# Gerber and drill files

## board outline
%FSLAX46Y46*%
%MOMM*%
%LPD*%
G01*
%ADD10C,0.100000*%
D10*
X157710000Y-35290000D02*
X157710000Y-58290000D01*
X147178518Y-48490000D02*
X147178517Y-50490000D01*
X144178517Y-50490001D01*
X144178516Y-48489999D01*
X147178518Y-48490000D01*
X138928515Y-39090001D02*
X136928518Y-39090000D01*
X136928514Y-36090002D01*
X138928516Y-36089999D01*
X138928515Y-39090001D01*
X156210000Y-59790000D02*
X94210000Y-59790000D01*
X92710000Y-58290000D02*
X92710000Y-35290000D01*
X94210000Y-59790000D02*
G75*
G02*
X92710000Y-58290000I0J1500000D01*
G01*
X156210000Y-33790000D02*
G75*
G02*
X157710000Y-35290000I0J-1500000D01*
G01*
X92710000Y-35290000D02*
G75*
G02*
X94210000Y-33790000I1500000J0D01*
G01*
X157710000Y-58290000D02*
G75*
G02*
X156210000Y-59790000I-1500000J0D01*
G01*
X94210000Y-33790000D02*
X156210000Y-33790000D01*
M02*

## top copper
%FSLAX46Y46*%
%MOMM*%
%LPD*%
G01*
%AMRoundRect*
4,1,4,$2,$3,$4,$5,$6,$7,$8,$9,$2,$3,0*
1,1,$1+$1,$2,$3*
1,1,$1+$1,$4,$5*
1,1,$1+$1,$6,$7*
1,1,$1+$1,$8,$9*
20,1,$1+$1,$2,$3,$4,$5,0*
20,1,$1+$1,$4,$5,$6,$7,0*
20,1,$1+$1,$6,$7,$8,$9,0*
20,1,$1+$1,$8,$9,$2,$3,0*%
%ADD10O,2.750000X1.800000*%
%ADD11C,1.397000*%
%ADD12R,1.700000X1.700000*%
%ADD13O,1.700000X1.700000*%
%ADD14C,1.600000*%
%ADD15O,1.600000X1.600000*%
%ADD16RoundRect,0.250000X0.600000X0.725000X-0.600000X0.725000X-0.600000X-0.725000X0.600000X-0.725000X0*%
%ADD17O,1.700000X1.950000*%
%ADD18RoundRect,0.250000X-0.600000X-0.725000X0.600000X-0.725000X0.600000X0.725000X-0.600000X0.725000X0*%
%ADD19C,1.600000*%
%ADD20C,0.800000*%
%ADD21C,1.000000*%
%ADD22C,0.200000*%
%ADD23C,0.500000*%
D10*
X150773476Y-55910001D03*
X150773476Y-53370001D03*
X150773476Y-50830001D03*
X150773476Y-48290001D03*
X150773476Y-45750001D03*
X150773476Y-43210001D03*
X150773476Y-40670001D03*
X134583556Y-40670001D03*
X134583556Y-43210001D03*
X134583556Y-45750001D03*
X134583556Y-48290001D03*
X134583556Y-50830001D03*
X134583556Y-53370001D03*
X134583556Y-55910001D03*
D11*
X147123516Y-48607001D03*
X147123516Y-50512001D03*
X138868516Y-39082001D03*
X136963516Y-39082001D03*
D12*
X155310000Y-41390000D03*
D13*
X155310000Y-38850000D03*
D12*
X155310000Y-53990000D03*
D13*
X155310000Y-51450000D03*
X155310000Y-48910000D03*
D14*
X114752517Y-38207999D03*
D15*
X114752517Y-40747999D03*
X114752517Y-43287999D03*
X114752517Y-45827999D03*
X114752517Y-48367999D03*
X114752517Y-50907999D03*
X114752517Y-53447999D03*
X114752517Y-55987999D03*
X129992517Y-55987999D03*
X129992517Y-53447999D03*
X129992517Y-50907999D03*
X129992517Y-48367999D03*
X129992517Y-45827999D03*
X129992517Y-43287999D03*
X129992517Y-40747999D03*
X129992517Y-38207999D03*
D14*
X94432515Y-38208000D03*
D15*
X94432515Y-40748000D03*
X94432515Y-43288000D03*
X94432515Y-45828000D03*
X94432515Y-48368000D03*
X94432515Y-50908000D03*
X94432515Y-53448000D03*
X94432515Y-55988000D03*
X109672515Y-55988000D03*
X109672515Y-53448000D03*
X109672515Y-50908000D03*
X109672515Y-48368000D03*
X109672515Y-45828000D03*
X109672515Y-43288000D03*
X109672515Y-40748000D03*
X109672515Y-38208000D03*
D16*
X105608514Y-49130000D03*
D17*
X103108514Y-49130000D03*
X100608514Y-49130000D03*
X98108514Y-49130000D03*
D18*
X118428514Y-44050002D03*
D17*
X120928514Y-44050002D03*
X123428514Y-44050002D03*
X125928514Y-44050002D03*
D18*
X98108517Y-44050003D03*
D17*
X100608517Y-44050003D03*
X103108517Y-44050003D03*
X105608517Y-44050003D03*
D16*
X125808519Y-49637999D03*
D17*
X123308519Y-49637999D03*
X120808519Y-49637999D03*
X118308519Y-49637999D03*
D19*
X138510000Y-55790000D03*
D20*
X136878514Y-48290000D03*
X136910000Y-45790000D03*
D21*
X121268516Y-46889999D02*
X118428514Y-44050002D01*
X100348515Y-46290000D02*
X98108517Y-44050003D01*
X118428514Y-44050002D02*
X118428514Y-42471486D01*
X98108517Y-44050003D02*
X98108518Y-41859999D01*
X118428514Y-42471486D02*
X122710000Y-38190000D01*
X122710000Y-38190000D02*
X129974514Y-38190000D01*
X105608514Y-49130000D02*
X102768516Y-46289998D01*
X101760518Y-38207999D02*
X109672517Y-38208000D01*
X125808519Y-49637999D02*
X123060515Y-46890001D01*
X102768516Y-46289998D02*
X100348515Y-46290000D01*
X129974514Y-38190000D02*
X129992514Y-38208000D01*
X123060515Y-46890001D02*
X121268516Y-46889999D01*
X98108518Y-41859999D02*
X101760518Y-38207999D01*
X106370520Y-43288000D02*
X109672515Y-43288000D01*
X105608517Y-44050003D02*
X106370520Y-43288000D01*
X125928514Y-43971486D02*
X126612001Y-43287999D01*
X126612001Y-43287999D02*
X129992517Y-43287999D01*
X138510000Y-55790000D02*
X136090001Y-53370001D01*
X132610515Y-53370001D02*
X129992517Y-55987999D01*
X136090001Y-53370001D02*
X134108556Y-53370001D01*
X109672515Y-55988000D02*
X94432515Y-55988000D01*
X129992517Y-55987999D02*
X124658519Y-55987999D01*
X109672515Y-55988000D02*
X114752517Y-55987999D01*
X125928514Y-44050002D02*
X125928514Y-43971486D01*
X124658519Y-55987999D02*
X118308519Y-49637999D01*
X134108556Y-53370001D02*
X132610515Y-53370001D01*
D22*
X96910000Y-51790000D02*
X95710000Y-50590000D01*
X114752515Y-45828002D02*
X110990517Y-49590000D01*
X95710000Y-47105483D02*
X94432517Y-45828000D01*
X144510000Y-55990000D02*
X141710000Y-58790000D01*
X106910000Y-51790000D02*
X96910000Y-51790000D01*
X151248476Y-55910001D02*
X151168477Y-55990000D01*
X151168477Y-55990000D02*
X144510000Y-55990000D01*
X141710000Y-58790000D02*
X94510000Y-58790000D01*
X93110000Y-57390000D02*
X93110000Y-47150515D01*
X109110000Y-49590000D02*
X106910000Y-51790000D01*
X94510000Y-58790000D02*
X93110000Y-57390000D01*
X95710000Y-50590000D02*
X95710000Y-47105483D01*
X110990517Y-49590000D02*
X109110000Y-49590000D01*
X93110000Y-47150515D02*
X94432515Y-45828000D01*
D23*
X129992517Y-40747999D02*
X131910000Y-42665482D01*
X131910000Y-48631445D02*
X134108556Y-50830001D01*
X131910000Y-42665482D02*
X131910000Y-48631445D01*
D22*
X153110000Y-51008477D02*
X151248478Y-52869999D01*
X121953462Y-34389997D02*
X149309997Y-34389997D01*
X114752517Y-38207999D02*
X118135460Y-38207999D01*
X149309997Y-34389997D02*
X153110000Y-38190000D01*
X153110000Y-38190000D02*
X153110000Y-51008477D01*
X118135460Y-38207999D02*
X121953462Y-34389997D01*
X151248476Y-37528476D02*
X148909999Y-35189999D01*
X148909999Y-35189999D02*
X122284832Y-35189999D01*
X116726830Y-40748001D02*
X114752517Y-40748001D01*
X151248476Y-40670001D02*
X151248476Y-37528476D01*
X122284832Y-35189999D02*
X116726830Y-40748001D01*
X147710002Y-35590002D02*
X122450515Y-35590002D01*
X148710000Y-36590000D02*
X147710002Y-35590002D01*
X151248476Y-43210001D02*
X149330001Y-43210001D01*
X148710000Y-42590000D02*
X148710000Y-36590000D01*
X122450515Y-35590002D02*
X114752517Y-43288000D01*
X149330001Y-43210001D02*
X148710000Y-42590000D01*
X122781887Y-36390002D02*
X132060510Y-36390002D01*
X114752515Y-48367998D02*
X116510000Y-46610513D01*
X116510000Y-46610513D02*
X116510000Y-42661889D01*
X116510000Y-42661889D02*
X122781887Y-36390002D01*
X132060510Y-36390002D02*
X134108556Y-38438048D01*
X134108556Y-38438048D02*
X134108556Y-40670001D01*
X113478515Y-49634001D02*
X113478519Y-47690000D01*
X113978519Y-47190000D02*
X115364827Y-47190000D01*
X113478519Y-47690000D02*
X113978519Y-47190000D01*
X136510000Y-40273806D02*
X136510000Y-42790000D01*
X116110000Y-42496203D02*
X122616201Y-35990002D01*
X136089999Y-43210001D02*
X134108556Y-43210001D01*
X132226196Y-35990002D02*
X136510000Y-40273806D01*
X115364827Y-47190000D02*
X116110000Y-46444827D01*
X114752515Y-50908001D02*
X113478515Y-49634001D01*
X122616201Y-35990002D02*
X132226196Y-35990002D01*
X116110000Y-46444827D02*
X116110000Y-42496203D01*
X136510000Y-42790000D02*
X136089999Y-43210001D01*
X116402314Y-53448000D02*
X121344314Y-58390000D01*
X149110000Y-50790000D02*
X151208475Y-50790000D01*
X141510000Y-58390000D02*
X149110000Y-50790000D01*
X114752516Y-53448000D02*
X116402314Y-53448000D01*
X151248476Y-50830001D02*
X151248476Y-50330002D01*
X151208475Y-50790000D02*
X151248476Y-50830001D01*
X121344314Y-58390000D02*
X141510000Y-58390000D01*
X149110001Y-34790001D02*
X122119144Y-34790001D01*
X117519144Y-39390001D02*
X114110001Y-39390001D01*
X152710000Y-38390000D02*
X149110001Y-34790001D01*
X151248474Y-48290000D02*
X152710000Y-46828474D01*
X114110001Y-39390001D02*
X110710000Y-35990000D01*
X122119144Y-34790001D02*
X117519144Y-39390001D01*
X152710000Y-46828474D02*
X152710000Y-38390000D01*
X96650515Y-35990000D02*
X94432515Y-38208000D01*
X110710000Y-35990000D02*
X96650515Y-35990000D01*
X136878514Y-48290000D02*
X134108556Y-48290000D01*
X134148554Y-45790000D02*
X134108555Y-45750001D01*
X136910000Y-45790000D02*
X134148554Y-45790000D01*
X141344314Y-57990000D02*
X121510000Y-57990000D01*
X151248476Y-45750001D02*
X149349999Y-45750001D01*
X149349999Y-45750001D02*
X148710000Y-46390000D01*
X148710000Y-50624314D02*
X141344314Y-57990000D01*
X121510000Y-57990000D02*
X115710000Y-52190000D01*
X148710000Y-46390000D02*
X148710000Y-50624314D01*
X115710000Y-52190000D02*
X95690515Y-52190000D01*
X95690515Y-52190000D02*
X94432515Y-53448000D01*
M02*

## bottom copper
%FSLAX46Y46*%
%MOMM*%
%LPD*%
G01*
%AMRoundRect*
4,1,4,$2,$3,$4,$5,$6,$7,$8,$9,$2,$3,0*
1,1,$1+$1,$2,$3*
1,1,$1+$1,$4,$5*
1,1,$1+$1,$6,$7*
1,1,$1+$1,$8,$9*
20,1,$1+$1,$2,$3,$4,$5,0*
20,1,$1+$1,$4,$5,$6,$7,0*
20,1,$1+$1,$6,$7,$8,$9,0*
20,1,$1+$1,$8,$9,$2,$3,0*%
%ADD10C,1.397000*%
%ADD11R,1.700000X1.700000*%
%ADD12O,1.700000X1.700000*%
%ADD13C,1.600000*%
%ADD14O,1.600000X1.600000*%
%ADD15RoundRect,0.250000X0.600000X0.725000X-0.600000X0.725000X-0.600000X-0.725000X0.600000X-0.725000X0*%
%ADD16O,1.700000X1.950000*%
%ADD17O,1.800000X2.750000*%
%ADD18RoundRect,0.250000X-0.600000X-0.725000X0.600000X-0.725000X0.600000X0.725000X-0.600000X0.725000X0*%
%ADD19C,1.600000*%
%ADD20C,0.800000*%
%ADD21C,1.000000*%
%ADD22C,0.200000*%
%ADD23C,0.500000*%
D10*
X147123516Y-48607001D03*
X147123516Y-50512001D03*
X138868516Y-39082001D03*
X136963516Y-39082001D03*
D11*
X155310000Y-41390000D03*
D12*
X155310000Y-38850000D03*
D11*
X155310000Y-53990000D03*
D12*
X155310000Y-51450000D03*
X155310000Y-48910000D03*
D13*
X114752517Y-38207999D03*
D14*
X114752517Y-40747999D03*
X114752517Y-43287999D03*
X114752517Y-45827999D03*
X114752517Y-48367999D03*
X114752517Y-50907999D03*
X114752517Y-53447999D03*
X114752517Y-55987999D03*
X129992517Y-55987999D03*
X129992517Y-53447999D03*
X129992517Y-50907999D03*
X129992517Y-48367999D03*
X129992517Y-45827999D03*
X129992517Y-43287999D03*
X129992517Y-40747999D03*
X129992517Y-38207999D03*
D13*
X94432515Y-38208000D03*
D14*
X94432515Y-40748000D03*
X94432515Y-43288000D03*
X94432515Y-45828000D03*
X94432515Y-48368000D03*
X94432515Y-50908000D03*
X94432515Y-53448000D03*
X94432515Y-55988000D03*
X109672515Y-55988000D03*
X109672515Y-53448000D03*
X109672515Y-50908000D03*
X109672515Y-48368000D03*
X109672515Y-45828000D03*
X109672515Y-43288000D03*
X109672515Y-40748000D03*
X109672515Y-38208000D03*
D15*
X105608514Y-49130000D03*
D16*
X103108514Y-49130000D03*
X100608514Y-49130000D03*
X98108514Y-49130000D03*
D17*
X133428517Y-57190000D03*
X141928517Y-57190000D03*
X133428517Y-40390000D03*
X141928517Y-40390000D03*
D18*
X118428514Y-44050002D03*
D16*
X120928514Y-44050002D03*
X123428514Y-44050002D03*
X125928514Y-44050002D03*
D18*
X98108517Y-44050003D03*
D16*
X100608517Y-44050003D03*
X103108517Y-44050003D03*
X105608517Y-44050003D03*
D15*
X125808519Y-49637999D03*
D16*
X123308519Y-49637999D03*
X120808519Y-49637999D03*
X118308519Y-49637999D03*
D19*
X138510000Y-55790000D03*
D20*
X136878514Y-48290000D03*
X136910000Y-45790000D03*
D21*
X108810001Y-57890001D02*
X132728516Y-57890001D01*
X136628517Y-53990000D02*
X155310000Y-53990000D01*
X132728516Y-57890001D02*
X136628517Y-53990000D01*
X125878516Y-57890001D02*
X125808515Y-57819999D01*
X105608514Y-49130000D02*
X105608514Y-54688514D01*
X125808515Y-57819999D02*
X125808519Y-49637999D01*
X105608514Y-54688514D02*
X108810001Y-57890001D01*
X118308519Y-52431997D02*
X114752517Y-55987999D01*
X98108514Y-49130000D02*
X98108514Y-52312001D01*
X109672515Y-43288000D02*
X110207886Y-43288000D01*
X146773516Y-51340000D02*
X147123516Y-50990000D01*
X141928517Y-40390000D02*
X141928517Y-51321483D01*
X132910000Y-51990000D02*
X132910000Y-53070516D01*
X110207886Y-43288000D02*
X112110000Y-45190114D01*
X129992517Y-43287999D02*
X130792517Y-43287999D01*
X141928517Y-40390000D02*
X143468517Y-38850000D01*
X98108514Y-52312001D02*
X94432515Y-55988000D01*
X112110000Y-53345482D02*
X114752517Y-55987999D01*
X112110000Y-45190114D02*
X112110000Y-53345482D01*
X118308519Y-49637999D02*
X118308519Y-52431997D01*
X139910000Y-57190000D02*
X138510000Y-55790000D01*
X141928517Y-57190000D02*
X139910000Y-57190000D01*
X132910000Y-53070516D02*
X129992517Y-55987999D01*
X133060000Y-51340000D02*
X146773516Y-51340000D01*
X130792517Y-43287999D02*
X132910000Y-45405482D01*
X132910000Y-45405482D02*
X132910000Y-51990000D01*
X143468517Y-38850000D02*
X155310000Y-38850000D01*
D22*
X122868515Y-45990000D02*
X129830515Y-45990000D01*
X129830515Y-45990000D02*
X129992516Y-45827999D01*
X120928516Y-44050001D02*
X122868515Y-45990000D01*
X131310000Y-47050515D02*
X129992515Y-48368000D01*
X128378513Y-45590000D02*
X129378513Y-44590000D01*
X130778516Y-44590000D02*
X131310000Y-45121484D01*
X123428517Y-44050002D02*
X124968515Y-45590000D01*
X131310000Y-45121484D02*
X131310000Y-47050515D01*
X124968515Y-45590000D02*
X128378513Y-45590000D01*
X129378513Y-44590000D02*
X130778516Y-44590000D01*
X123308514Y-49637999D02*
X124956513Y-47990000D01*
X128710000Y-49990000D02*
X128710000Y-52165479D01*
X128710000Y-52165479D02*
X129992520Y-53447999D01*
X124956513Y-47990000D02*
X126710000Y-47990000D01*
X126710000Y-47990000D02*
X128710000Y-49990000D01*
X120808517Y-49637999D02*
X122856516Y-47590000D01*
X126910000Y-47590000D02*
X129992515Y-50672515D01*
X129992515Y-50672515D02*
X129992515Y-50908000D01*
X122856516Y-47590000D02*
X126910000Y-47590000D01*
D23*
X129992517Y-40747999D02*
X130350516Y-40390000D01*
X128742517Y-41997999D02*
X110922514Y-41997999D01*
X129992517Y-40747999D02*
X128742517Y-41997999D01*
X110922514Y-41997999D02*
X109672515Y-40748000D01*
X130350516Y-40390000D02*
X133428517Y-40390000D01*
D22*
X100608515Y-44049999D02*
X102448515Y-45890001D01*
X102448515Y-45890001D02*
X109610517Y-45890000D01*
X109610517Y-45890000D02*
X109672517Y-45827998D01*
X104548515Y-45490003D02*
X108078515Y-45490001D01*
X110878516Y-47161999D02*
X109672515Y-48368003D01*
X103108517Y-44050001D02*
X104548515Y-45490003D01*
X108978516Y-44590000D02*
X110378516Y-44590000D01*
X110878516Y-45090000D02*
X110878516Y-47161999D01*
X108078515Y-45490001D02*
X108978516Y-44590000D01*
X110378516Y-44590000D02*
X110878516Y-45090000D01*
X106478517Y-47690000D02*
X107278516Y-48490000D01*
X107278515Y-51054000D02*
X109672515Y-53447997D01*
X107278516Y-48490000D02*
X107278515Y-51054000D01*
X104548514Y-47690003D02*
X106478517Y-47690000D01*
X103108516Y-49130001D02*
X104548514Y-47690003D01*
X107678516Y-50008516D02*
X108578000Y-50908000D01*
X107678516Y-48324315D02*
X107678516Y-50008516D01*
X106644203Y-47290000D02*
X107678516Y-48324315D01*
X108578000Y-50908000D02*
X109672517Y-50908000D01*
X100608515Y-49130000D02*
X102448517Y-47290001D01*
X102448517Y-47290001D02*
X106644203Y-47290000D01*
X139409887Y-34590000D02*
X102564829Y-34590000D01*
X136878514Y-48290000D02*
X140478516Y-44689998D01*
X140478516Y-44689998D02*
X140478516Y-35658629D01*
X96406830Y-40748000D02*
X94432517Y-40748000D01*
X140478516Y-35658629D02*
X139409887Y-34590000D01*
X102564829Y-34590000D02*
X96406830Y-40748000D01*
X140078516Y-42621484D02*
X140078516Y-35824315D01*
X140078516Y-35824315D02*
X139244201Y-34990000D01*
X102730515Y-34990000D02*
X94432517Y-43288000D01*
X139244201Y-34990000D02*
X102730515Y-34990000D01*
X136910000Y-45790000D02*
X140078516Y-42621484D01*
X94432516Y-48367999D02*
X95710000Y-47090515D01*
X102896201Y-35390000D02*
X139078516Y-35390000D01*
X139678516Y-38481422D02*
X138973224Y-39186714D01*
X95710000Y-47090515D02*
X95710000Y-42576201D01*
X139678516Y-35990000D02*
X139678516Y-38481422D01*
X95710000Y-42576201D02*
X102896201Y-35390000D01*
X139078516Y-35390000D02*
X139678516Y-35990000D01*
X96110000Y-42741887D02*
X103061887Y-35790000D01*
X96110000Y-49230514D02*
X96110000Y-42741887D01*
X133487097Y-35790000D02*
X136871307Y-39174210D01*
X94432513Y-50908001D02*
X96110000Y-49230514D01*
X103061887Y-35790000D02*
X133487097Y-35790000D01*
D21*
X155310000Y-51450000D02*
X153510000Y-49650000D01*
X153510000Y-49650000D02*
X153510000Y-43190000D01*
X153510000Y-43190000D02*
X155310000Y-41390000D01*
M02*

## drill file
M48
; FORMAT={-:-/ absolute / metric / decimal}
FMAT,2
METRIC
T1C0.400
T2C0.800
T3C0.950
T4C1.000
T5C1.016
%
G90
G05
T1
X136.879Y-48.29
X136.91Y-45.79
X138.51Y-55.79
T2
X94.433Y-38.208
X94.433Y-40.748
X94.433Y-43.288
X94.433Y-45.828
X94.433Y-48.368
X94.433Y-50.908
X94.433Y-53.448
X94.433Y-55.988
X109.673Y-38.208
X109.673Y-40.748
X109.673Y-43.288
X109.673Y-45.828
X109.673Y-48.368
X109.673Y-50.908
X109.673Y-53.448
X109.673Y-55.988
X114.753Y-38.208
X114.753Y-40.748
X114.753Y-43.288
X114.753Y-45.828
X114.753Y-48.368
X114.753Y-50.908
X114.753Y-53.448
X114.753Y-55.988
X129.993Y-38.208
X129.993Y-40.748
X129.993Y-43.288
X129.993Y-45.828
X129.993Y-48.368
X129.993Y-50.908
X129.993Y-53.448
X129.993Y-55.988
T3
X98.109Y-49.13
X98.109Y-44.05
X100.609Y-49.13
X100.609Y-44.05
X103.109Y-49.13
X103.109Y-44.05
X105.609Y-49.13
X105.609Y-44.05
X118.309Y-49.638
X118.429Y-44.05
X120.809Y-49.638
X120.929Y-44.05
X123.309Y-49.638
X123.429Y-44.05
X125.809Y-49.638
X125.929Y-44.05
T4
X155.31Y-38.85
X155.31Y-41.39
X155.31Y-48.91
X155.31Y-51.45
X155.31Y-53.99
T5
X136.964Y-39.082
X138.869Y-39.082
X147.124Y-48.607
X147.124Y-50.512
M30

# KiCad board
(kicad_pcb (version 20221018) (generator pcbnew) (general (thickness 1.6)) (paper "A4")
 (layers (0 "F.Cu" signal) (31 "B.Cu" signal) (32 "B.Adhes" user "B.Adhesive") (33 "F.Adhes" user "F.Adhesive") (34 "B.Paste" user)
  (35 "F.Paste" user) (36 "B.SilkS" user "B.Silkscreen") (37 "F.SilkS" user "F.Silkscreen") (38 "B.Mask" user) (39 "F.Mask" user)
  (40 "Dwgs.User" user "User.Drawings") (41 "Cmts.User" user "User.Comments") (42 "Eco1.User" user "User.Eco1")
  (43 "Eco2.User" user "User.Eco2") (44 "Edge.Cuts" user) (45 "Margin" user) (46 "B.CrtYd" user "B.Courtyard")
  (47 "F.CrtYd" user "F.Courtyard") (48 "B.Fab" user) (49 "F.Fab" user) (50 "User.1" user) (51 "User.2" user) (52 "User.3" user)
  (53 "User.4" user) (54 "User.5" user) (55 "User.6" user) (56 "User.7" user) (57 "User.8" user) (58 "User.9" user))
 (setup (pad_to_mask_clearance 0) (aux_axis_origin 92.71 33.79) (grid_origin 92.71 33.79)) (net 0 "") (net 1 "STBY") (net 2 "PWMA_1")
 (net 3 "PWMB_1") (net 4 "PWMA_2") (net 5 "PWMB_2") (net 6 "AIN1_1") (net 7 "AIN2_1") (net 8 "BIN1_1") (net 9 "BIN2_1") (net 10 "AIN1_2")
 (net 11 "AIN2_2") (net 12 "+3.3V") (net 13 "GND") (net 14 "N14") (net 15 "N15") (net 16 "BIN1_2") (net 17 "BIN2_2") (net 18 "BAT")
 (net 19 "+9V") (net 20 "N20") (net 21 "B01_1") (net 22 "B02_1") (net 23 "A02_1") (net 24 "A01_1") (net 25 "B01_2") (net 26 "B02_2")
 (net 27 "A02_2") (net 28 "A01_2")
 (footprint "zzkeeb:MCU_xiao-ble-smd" (layer "F.Cu") (at 142.678516 48.290001 180)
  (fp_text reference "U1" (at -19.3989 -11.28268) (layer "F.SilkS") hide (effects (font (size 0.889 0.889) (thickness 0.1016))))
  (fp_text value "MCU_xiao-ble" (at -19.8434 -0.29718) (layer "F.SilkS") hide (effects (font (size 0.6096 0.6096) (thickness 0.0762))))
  (pad "1" smd oval (at -8.56996 -7.62) (size 2.75 1.8) (drill (offset -0.475 0)) (layers "F.Cu" "F.Paste" "F.Mask") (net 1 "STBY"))
  (pad "2" smd oval (at -8.56996 -5.08) (size 2.75 1.8) (drill (offset -0.475 0)) (layers "F.Cu" "F.Paste" "F.Mask") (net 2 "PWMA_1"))
  (pad "3" smd oval (at -8.56996 -2.54) (size 2.75 1.8) (drill (offset -0.475 0)) (layers "F.Cu" "F.Paste" "F.Mask") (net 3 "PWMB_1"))
  (pad "4" smd oval (at -8.56996 0) (size 2.75 1.8) (drill (offset -0.475 0)) (layers "F.Cu" "F.Paste" "F.Mask") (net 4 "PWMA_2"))
  (pad "5" smd oval (at -8.56996 2.54) (size 2.75 1.8) (drill (offset -0.475 0)) (layers "F.Cu" "F.Paste" "F.Mask") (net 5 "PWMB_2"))
  (pad "6" smd oval (at -8.56996 5.08) (size 2.75 1.8) (drill (offset -0.475 0)) (layers "F.Cu" "F.Paste" "F.Mask") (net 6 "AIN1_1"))
  (pad "7" smd oval (at -8.56996 7.62) (size 2.75 1.8) (drill (offset -0.475 0)) (layers "F.Cu" "F.Paste" "F.Mask") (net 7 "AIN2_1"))
  (pad "8" smd oval (at 8.56996 7.62 180) (size 2.75 1.8) (drill (offset -0.475 0)) (layers "F.Cu" "F.Paste" "F.Mask") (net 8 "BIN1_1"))
  (pad "9" smd oval (at 8.56996 5.08 180) (size 2.75 1.8) (drill (offset -0.475 0)) (layers "F.Cu" "F.Paste" "F.Mask") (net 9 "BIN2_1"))
  (pad "10" smd oval (at 8.56996 2.54 180) (size 2.75 1.8) (drill (offset -0.475 0)) (layers "F.Cu" "F.Paste" "F.Mask") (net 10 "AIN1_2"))
  (pad "11" smd oval (at 8.56996 0 180) (size 2.75 1.8) (drill (offset -0.475 0)) (layers "F.Cu" "F.Paste" "F.Mask") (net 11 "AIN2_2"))
  (pad "12" smd oval (at 8.56996 -2.54 180) (size 2.75 1.8) (drill (offset -0.475 0)) (layers "F.Cu" "F.Paste" "F.Mask") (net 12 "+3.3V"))
  (pad "13" smd oval (at 8.56996 -5.08 180) (size 2.75 1.8) (drill (offset -0.475 0)) (layers "F.Cu" "F.Paste" "F.Mask") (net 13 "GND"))
  (pad "14" smd oval (at 8.56996 -7.62 180) (size 2.75 1.8) (drill (offset -0.475 0)) (layers "F.Cu" "F.Paste" "F.Mask") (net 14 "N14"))
  (pad "19" thru_hole circle (at -4.445 -0.317) (size 1.397 1.397) (drill 1.016) (layers "*.Cu" "*.Mask") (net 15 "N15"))
  (pad "20" thru_hole circle (at -4.445 -2.222) (size 1.397 1.397) (drill 1.016) (layers "*.Cu" "*.Mask") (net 13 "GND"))
  (pad "21" thru_hole circle (at 3.81 9.208) (size 1.397 1.397) (drill 1.016) (layers "*.Cu" "*.Mask") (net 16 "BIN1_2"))
  (pad "22" thru_hole circle (at 5.715 9.208) (size 1.397 1.397) (drill 1.016) (layers "*.Cu" "*.Mask") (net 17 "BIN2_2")))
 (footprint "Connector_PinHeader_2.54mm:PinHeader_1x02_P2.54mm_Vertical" (layer "F.Cu") (at 155.31 41.39 180)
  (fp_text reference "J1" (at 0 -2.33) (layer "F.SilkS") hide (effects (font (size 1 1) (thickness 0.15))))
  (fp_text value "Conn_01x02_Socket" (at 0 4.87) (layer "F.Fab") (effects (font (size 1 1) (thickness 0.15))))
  (pad "1" thru_hole rect (at 0 0 180) (size 1.7 1.7) (drill 1) (layers "*.Cu" "*.Mask") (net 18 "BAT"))
  (pad "2" thru_hole oval (at 0 2.54 180) (size 1.7 1.7) (drill 1) (layers "*.Cu" "*.Mask") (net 13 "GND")))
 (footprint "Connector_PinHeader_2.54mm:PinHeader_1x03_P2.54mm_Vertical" (layer "F.Cu") (at 155.31 53.99 180)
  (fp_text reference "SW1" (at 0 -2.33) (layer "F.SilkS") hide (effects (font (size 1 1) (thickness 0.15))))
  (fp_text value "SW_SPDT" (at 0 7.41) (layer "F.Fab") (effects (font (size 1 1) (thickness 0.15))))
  (pad "1" thru_hole rect (at 0 0 180) (size 1.7 1.7) (drill 1) (layers "*.Cu" "*.Mask") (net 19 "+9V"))
  (pad "2" thru_hole oval (at 0 2.54 180) (size 1.7 1.7) (drill 1) (layers "*.Cu" "*.Mask") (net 18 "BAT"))
  (pad "3" thru_hole oval (at 0 5.08 180) (size 1.7 1.7) (drill 1) (layers "*.Cu" "*.Mask") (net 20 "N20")))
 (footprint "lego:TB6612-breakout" (layer "F.Cu") (at 114.752517 38.207999)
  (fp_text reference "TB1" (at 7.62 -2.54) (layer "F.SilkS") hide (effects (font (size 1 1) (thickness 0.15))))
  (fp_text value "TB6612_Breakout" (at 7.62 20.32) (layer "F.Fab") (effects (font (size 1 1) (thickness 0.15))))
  (pad "1" thru_hole circle (at 0 0) (size 1.6 1.6) (drill 0.8) (layers "*.Cu" "*.Mask") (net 2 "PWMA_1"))
  (pad "2" thru_hole oval (at 0 2.54) (size 1.6 1.6) (drill 0.8) (layers "*.Cu" "*.Mask") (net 7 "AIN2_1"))
  (pad "3" thru_hole oval (at 0 5.08) (size 1.6 1.6) (drill 0.8) (layers "*.Cu" "*.Mask") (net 6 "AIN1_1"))
  (pad "4" thru_hole oval (at 0 7.62) (size 1.6 1.6) (drill 0.8) (layers "*.Cu" "*.Mask") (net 1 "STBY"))
  (pad "5" thru_hole oval (at 0 10.16) (size 1.6 1.6) (drill 0.8) (layers "*.Cu" "*.Mask") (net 8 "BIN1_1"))
  (pad "6" thru_hole oval (at 0 12.7) (size 1.6 1.6) (drill 0.8) (layers "*.Cu" "*.Mask") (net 9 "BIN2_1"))
  (pad "7" thru_hole oval (at 0 15.24) (size 1.6 1.6) (drill 0.8) (layers "*.Cu" "*.Mask") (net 3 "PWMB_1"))
  (pad "8" thru_hole oval (at 0 17.78) (size 1.6 1.6) (drill 0.8) (layers "*.Cu" "*.Mask") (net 13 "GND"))
  (pad "9" thru_hole oval (at 15.24 17.78) (size 1.6 1.6) (drill 0.8) (layers "*.Cu" "*.Mask") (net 13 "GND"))
  (pad "10" thru_hole oval (at 15.24 15.24) (size 1.6 1.6) (drill 0.8) (layers "*.Cu" "*.Mask") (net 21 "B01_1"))
  (pad "11" thru_hole oval (at 15.24 12.7) (size 1.6 1.6) (drill 0.8) (layers "*.Cu" "*.Mask") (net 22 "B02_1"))
  (pad "12" thru_hole oval (at 15.24 10.16) (size 1.6 1.6) (drill 0.8) (layers "*.Cu" "*.Mask") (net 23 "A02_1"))
  (pad "13" thru_hole oval (at 15.24 7.62) (size 1.6 1.6) (drill 0.8) (layers "*.Cu" "*.Mask") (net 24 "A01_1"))
  (pad "14" thru_hole oval (at 15.24 5.08) (size 1.6 1.6) (drill 0.8) (layers "*.Cu" "*.Mask") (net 13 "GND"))
  (pad "15" thru_hole oval (at 15.24 2.54) (size 1.6 1.6) (drill 0.8) (layers "*.Cu" "*.Mask") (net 12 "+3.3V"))
  (pad "16" thru_hole oval (at 15.24 0) (size 1.6 1.6) (drill 0.8) (layers "*.Cu" "*.Mask") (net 19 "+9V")))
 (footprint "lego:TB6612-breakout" (layer "F.Cu") (at 94.432515 38.208)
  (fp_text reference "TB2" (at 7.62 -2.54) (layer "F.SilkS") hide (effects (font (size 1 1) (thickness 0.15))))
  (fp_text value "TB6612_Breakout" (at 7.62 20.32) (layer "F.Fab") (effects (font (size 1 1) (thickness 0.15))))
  (pad "1" thru_hole circle (at 0 0) (size 1.6 1.6) (drill 0.8) (layers "*.Cu" "*.Mask") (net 4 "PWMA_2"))
  (pad "2" thru_hole oval (at 0 2.54) (size 1.6 1.6) (drill 0.8) (layers "*.Cu" "*.Mask") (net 11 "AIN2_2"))
  (pad "3" thru_hole oval (at 0 5.08) (size 1.6 1.6) (drill 0.8) (layers "*.Cu" "*.Mask") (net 10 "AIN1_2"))
  (pad "4" thru_hole oval (at 0 7.62) (size 1.6 1.6) (drill 0.8) (layers "*.Cu" "*.Mask") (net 1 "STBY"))
  (pad "5" thru_hole oval (at 0 10.16) (size 1.6 1.6) (drill 0.8) (layers "*.Cu" "*.Mask") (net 16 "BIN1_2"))
  (pad "6" thru_hole oval (at 0 12.7) (size 1.6 1.6) (drill 0.8) (layers "*.Cu" "*.Mask") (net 17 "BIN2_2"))
  (pad "7" thru_hole oval (at 0 15.24) (size 1.6 1.6) (drill 0.8) (layers "*.Cu" "*.Mask") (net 5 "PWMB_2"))
  (pad "8" thru_hole oval (at 0 17.78) (size 1.6 1.6) (drill 0.8) (layers "*.Cu" "*.Mask") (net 13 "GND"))
  (pad "9" thru_hole oval (at 15.24 17.78) (size 1.6 1.6) (drill 0.8) (layers "*.Cu" "*.Mask") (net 13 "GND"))
  (pad "10" thru_hole oval (at 15.24 15.24) (size 1.6 1.6) (drill 0.8) (layers "*.Cu" "*.Mask") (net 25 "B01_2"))
  (pad "11" thru_hole oval (at 15.24 12.7) (size 1.6 1.6) (drill 0.8) (layers "*.Cu" "*.Mask") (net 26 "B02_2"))
  (pad "12" thru_hole oval (at 15.24 10.16) (size 1.6 1.6) (drill 0.8) (layers "*.Cu" "*.Mask") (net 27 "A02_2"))
  (pad "13" thru_hole oval (at 15.24 7.62) (size 1.6 1.6) (drill 0.8) (layers "*.Cu" "*.Mask") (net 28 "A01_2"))
  (pad "14" thru_hole oval (at 15.24 5.08) (size 1.6 1.6) (drill 0.8) (layers "*.Cu" "*.Mask") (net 13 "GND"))
  (pad "15" thru_hole oval (at 15.24 2.54) (size 1.6 1.6) (drill 0.8) (layers "*.Cu" "*.Mask") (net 12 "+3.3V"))
  (pad "16" thru_hole oval (at 15.24 0) (size 1.6 1.6) (drill 0.8) (layers "*.Cu" "*.Mask") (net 19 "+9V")))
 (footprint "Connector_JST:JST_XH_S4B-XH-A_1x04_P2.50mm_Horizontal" (layer "B.Cu") (at 105.608514 49.13 180)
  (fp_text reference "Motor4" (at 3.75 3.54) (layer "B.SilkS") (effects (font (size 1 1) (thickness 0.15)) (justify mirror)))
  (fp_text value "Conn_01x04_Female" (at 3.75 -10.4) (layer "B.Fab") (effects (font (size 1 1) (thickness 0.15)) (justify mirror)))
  (pad "1" thru_hole roundrect (at 0 0 180) (size 1.7 1.95) (drill 0.95) (layers "*.Cu" "*.Mask") (roundrect_rratio 0.1470588235)
   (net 19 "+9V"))
  (pad "2" thru_hole oval (at 2.5 0 180) (size 1.7 1.95) (drill 0.95) (layers "*.Cu" "*.Mask") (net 25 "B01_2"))
  (pad "3" thru_hole oval (at 5 0 180) (size 1.7 1.95) (drill 0.95) (layers "*.Cu" "*.Mask") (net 26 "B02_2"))
  (pad "4" thru_hole oval (at 7.5 0 180) (size 1.7 1.95) (drill 0.95) (layers "*.Cu" "*.Mask") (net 13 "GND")))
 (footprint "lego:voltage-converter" (layer "B.Cu") (at 137.678517 48.79 -90)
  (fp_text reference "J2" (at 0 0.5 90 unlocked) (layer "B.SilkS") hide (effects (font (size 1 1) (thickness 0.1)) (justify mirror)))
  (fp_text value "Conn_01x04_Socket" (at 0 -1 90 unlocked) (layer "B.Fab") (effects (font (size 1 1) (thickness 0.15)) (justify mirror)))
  (pad "1" smd oval (at 8.4 4.25 270) (size 2.75 1.8) (layers "B.Cu" "B.Paste" "B.Mask") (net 19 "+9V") (thermal_bridge_angle 45))
  (pad "2" smd oval (at 8.4 -4.25 270) (size 2.75 1.8) (layers "B.Cu" "B.Paste" "B.Mask") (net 13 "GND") (thermal_bridge_angle 45))
  (pad "3" smd oval (at -8.4 4.25 270) (size 2.75 1.8) (layers "B.Cu" "B.Paste" "B.Mask") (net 12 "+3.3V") (thermal_bridge_angle 45))
  (pad "4" smd oval (at -8.4 -4.25 270) (size 2.75 1.8) (layers "B.Cu" "B.Paste" "B.Mask") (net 13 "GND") (thermal_bridge_angle 45)))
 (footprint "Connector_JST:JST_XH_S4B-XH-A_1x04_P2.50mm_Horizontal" (layer "B.Cu") (at 118.428514 44.050002)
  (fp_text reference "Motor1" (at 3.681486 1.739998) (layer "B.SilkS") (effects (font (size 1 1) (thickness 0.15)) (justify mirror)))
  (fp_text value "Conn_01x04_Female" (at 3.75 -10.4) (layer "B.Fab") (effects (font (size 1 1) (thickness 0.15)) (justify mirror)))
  (pad "1" thru_hole roundrect (at 0 0) (size 1.7 1.95) (drill 0.95) (layers "*.Cu" "*.Mask") (roundrect_rratio 0.1470588235) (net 19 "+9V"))
  (pad "2" thru_hole oval (at 2.5 0) (size 1.7 1.95) (drill 0.95) (layers "*.Cu" "*.Mask") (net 24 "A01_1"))
  (pad "3" thru_hole oval (at 5 0) (size 1.7 1.95) (drill 0.95) (layers "*.Cu" "*.Mask") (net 23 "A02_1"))
  (pad "4" thru_hole oval (at 7.5 0) (size 1.7 1.95) (drill 0.95) (layers "*.Cu" "*.Mask") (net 13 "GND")))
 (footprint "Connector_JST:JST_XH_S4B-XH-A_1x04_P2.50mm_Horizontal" (layer "B.Cu") (at 98.108517 44.050003)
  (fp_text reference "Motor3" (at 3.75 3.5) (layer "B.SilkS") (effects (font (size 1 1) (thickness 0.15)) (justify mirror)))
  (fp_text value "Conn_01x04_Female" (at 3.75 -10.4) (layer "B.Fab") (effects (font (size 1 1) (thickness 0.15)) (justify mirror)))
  (pad "1" thru_hole roundrect (at 0 0) (size 1.7 1.95) (drill 0.95) (layers "*.Cu" "*.Mask") (roundrect_rratio 0.1470588235) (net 19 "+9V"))
  (pad "2" thru_hole oval (at 2.5 0) (size 1.7 1.95) (drill 0.95) (layers "*.Cu" "*.Mask") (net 28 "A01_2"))
  (pad "3" thru_hole oval (at 5 0) (size 1.7 1.95) (drill 0.95) (layers "*.Cu" "*.Mask") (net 27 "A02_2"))
  (pad "4" thru_hole oval (at 7.5 0) (size 1.7 1.95) (drill 0.95) (layers "*.Cu" "*.Mask") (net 13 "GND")))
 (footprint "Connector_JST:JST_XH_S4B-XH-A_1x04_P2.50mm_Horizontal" (layer "B.Cu") (at 125.808519 49.637999 180)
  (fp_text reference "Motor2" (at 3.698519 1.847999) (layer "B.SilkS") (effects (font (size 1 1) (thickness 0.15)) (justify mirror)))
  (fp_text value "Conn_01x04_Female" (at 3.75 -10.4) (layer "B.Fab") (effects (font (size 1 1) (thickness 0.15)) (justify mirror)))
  (pad "1" thru_hole roundrect (at 0 0 180) (size 1.7 1.95) (drill 0.95) (layers "*.Cu" "*.Mask") (roundrect_rratio 0.1470588235)
   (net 19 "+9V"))
  (pad "2" thru_hole oval (at 2.5 0 180) (size 1.7 1.95) (drill 0.95) (layers "*.Cu" "*.Mask") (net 21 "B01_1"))
  (pad "3" thru_hole oval (at 5 0 180) (size 1.7 1.95) (drill 0.95) (layers "*.Cu" "*.Mask") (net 22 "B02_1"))
  (pad "4" thru_hole oval (at 7.5 0 180) (size 1.7 1.95) (drill 0.95) (layers "*.Cu" "*.Mask") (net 13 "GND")))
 (gr_line (start 157.71 35.29) (end 157.71 58.29) (stroke (width 0.1) (type default)) (layer "Edge.Cuts"))
 (gr_poly
  (pts (xy 147.178518 48.49) (xy 147.178517 50.49) (xy 144.178517 50.490001) (xy 144.178516 48.489999)) (stroke (width 0.1) (type default))
  (fill none) (layer "Edge.Cuts"))
 (gr_poly
  (pts (xy 138.928515 39.090001) (xy 136.928518 39.09) (xy 136.928514 36.090002) (xy 138.928516 36.089999))
  (stroke (width 0.1) (type default)) (fill none) (layer "Edge.Cuts"))
 (gr_line (start 156.21 59.79) (end 94.21 59.79) (stroke (width 0.1) (type default)) (layer "Edge.Cuts"))
 (gr_line (start 92.71 58.29) (end 92.71 35.29) (stroke (width 0.1) (type default)) (layer "Edge.Cuts"))
 (gr_arc (start 94.21 59.79) (mid 93.14934 59.35066) (end 92.71 58.29) (stroke (width 0.1) (type default)) (layer "Edge.Cuts"))
 (gr_arc (start 156.21 33.79) (mid 157.27066 34.22934) (end 157.71 35.29) (stroke (width 0.1) (type default)) (layer "Edge.Cuts"))
 (gr_arc (start 92.71 35.29) (mid 93.14934 34.22934) (end 94.21 33.79) (stroke (width 0.1) (type default)) (layer "Edge.Cuts"))
 (gr_arc (start 157.71 58.29) (mid 157.27066 59.35066) (end 156.21 59.79) (stroke (width 0.1) (type default)) (layer "Edge.Cuts"))
 (gr_line (start 94.21 33.79) (end 156.21 33.79) (stroke (width 0.1) (type default)) (layer "Edge.Cuts"))
 (segment (start 121.268516 46.889999) (end 118.428514 44.050002) (width 1) (layer "F.Cu") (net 19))
 (segment (start 100.348515 46.29) (end 98.108517 44.050003) (width 1) (layer "F.Cu") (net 19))
 (segment (start 118.428514 44.050002) (end 118.428514 42.471486) (width 1) (layer "F.Cu") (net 19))
 (segment (start 98.108517 44.050003) (end 98.108518 41.859999) (width 1) (layer "F.Cu") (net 19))
 (segment (start 118.428514 42.471486) (end 122.71 38.19) (width 1) (layer "F.Cu") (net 19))
 (segment (start 122.71 38.19) (end 129.974514 38.19) (width 1) (layer "F.Cu") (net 19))
 (segment (start 105.608514 49.13) (end 102.768516 46.289998) (width 1) (layer "F.Cu") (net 19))
 (segment (start 101.760518 38.207999) (end 109.672517 38.208) (width 1) (layer "F.Cu") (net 19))
 (segment (start 125.808519 49.637999) (end 123.060515 46.890001) (width 1) (layer "F.Cu") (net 19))
 (segment (start 102.768516 46.289998) (end 100.348515 46.29) (width 1) (layer "F.Cu") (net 19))
 (segment (start 129.974514 38.19) (end 129.992514 38.208) (width 1) (layer "F.Cu") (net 19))
 (segment (start 123.060515 46.890001) (end 121.268516 46.889999) (width 1) (layer "F.Cu") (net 19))
 (segment (start 98.108518 41.859999) (end 101.760518 38.207999) (width 1) (layer "F.Cu") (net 19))
 (segment (start 108.810001 57.890001) (end 132.728516 57.890001) (width 1) (layer "B.Cu") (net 19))
 (segment (start 136.628517 53.99) (end 155.31 53.99) (width 1) (layer "B.Cu") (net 19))
 (segment (start 132.728516 57.890001) (end 136.628517 53.99) (width 1) (layer "B.Cu") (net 19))
 (segment (start 125.878516 57.890001) (end 125.808515 57.819999) (width 1) (layer "B.Cu") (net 19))
 (segment (start 105.608514 49.13) (end 105.608514 54.688514) (width 1) (layer "B.Cu") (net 19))
 (segment (start 125.808515 57.819999) (end 125.808519 49.637999) (width 1) (layer "B.Cu") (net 19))
 (segment (start 105.608514 54.688514) (end 108.810001 57.890001) (width 1) (layer "B.Cu") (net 19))
 (segment (start 106.37052 43.288) (end 109.672515 43.288) (width 1) (layer "F.Cu") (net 13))
 (segment (start 105.608517 44.050003) (end 106.37052 43.288) (width 1) (layer "F.Cu") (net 13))
 (segment (start 125.928514 43.971486) (end 126.612001 43.287999) (width 1) (layer "F.Cu") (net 13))
 (segment (start 126.612001 43.287999) (end 129.992517 43.287999) (width 1) (layer "F.Cu") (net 13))
 (segment (start 138.51 55.79) (end 136.090001 53.370001) (width 1) (layer "F.Cu") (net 13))
 (segment (start 132.610515 53.370001) (end 129.992517 55.987999) (width 1) (layer "F.Cu") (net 13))
 (segment (start 136.090001 53.370001) (end 134.108556 53.370001) (width 1) (layer "F.Cu") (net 13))
 (segment (start 109.672515 55.988) (end 94.432515 55.988) (width 1) (layer "F.Cu") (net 13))
 (segment (start 129.992517 55.987999) (end 124.658519 55.987999) (width 1) (layer "F.Cu") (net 13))
 (segment (start 109.672515 55.988) (end 114.752517 55.987999) (width 1) (layer "F.Cu") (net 13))
 (segment (start 125.928514 44.050002) (end 125.928514 43.971486) (width 1) (layer "F.Cu") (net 13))
 (segment (start 124.658519 55.987999) (end 118.308519 49.637999) (width 1) (layer "F.Cu") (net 13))
 (segment (start 134.108556 53.370001) (end 132.610515 53.370001) (width 1) (layer "F.Cu") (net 13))
 (via (at 138.51 55.79) (size 1.6) (drill 0.4) (layers "F.Cu" "B.Cu") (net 13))
 (segment (start 118.308519 52.431997) (end 114.752517 55.987999) (width 1) (layer "B.Cu") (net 13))
 (segment (start 98.108514 49.13) (end 98.108514 52.312001) (width 1) (layer "B.Cu") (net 13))
 (segment (start 109.672515 43.288) (end 110.207886 43.288) (width 1) (layer "B.Cu") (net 13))
 (segment (start 146.773516 51.34) (end 147.123516 50.99) (width 1) (layer "B.Cu") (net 13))
 (segment (start 141.928517 40.39) (end 141.928517 51.321483) (width 1) (layer "B.Cu") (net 13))
 (segment (start 132.91 51.99) (end 132.91 53.070516) (width 1) (layer "B.Cu") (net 13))
 (segment (start 110.207886 43.288) (end 112.11 45.190114) (width 1) (layer "B.Cu") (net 13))
 (segment (start 129.992517 43.287999) (end 130.792517 43.287999) (width 1) (layer "B.Cu") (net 13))
 (segment (start 141.928517 40.39) (end 143.468517 38.85) (width 1) (layer "B.Cu") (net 13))
 (segment (start 98.108514 52.312001) (end 94.432515 55.988) (width 1) (layer "B.Cu") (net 13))
 (segment (start 112.11 53.345482) (end 114.752517 55.987999) (width 1) (layer "B.Cu") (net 13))
 (segment (start 112.11 45.190114) (end 112.11 53.345482) (width 1) (layer "B.Cu") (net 13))
 (segment (start 118.308519 49.637999) (end 118.308519 52.431997) (width 1) (layer "B.Cu") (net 13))
 (segment (start 139.91 57.19) (end 138.51 55.79) (width 1) (layer "B.Cu") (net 13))
 (segment (start 141.928517 57.19) (end 139.91 57.19) (width 1) (layer "B.Cu") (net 13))
 (segment (start 132.91 53.070516) (end 129.992517 55.987999) (width 1) (layer "B.Cu") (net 13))
 (segment (start 133.06 51.34) (end 146.773516 51.34) (width 1) (layer "B.Cu") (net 13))
 (segment (start 130.792517 43.287999) (end 132.91 45.405482) (width 1) (layer "B.Cu") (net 13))
 (segment (start 132.91 45.405482) (end 132.91 51.99) (width 1) (layer "B.Cu") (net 13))
 (segment (start 143.468517 38.85) (end 155.31 38.85) (width 1) (layer "B.Cu") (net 13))
 (segment (start 122.868515 45.99) (end 129.830515 45.99) (width 0.2) (layer "B.Cu") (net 24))
 (segment (start 129.830515 45.99) (end 129.992516 45.827999) (width 0.2) (layer "B.Cu") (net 24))
 (segment (start 120.928516 44.050001) (end 122.868515 45.99) (width 0.2) (layer "B.Cu") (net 24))
 (segment (start 131.31 47.050515) (end 129.992515 48.368) (width 0.2) (layer "B.Cu") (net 23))
 (segment (start 128.378513 45.59) (end 129.378513 44.59) (width 0.2) (layer "B.Cu") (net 23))
 (segment (start 130.778516 44.59) (end 131.31 45.121484) (width 0.2) (layer "B.Cu") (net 23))
 (segment (start 123.428517 44.050002) (end 124.968515 45.59) (width 0.2) (layer "B.Cu") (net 23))
 (segment (start 131.31 45.121484) (end 131.31 47.050515) (width 0.2) (layer "B.Cu") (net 23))
 (segment (start 124.968515 45.59) (end 128.378513 45.59) (width 0.2) (layer "B.Cu") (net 23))
 (segment (start 129.378513 44.59) (end 130.778516 44.59) (width 0.2) (layer "B.Cu") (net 23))
 (segment (start 123.308514 49.637999) (end 124.956513 47.99) (width 0.2) (layer "B.Cu") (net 21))
 (segment (start 128.71 49.99) (end 128.71 52.165479) (width 0.2) (layer "B.Cu") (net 21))
 (segment (start 128.71 52.165479) (end 129.99252 53.447999) (width 0.2) (layer "B.Cu") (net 21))
 (segment (start 124.956513 47.99) (end 126.71 47.99) (width 0.2) (layer "B.Cu") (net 21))
 (segment (start 126.71 47.99) (end 128.71 49.99) (width 0.2) (layer "B.Cu") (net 21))
 (segment (start 120.808517 49.637999) (end 122.856516 47.59) (width 0.2) (layer "B.Cu") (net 22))
 (segment (start 126.91 47.59) (end 129.992515 50.672515) (width 0.2) (layer "B.Cu") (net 22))
 (segment (start 129.992515 50.672515) (end 129.992515 50.908) (width 0.2) (layer "B.Cu") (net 22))
 (segment (start 122.856516 47.59) (end 126.91 47.59) (width 0.2) (layer "B.Cu") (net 22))
 (segment (start 96.91 51.79) (end 95.71 50.59) (width 0.2) (layer "F.Cu") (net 1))
 (segment (start 114.752515 45.828002) (end 110.990517 49.59) (width 0.2) (layer "F.Cu") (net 1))
 (segment (start 95.71 47.105483) (end 94.432517 45.828) (width 0.2) (layer "F.Cu") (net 1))
 (segment (start 144.51 55.99) (end 141.71 58.79) (width 0.2) (layer "F.Cu") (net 1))
 (segment (start 106.91 51.79) (end 96.91 51.79) (width 0.2) (layer "F.Cu") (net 1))
 (segment (start 151.248476 55.910001) (end 151.168477 55.99) (width 0.2) (layer "F.Cu") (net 1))
 (segment (start 151.168477 55.99) (end 144.51 55.99) (width 0.2) (layer "F.Cu") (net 1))
 (segment (start 141.71 58.79) (end 94.51 58.79) (width 0.2) (layer "F.Cu") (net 1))
 (segment (start 93.11 57.39) (end 93.11 47.150515) (width 0.2) (layer "F.Cu") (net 1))
 (segment (start 109.11 49.59) (end 106.91 51.79) (width 0.2) (layer "F.Cu") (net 1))
 (segment (start 94.51 58.79) (end 93.11 57.39) (width 0.2) (layer "F.Cu") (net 1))
 (segment (start 95.71 50.59) (end 95.71 47.105483) (width 0.2) (layer "F.Cu") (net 1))
 (segment (start 110.990517 49.59) (end 109.11 49.59) (width 0.2) (layer "F.Cu") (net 1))
 (segment (start 93.11 47.150515) (end 94.432515 45.828) (width 0.2) (layer "F.Cu") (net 1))
 (segment (start 129.992517 40.747999) (end 131.91 42.665482) (width 0.5) (layer "F.Cu") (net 12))
 (segment (start 131.91 48.631445) (end 134.108556 50.830001) (width 0.5) (layer "F.Cu") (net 12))
 (segment (start 131.91 42.665482) (end 131.91 48.631445) (width 0.5) (layer "F.Cu") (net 12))
 (segment (start 129.992517 40.747999) (end 130.350516 40.39) (width 0.5) (layer "B.Cu") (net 12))
 (segment (start 128.742517 41.997999) (end 110.922514 41.997999) (width 0.5) (layer "B.Cu") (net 12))
 (segment (start 129.992517 40.747999) (end 128.742517 41.997999) (width 0.5) (layer "B.Cu") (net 12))
 (segment (start 110.922514 41.997999) (end 109.672515 40.748) (width 0.5) (layer "B.Cu") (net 12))
 (segment (start 130.350516 40.39) (end 133.428517 40.39) (width 0.5) (layer "B.Cu") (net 12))
 (segment (start 100.608515 44.049999) (end 102.448515 45.890001) (width 0.2) (layer "B.Cu") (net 28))
 (segment (start 102.448515 45.890001) (end 109.610517 45.89) (width 0.2) (layer "B.Cu") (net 28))
 (segment (start 109.610517 45.89) (end 109.672517 45.827998) (width 0.2) (layer "B.Cu") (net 28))
 (segment (start 104.548515 45.490003) (end 108.078515 45.490001) (width 0.2) (layer "B.Cu") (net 27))
 (segment (start 110.878516 47.161999) (end 109.672515 48.368003) (width 0.2) (layer "B.Cu") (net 27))
 (segment (start 103.108517 44.050001) (end 104.548515 45.490003) (width 0.2) (layer "B.Cu") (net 27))
 (segment (start 108.978516 44.59) (end 110.378516 44.59) (width 0.2) (layer "B.Cu") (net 27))
 (segment (start 110.878516 45.09) (end 110.878516 47.161999) (width 0.2) (layer "B.Cu") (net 27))
 (segment (start 108.078515 45.490001) (end 108.978516 44.59) (width 0.2) (layer "B.Cu") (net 27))
 (segment (start 110.378516 44.59) (end 110.878516 45.09) (width 0.2) (layer "B.Cu") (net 27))
 (segment (start 106.478517 47.69) (end 107.278516 48.49) (width 0.2) (layer "B.Cu") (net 25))
 (segment (start 107.278515 51.054) (end 109.672515 53.447997) (width 0.2) (layer "B.Cu") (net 25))
 (segment (start 107.278516 48.49) (end 107.278515 51.054) (width 0.2) (layer "B.Cu") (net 25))
 (segment (start 104.548514 47.690003) (end 106.478517 47.69) (width 0.2) (layer "B.Cu") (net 25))
 (segment (start 103.108516 49.130001) (end 104.548514 47.690003) (width 0.2) (layer "B.Cu") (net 25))
 (segment (start 107.678516 50.008516) (end 108.578 50.908) (width 0.2) (layer "B.Cu") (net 26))
 (segment (start 107.678516 48.324315) (end 107.678516 50.008516) (width 0.2) (layer "B.Cu") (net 26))
 (segment (start 106.644203 47.29) (end 107.678516 48.324315) (width 0.2) (layer "B.Cu") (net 26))
 (segment (start 108.578 50.908) (end 109.672517 50.908) (width 0.2) (layer "B.Cu") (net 26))
 (segment (start 100.608515 49.13) (end 102.448517 47.290001) (width 0.2) (layer "B.Cu") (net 26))
 (segment (start 102.448517 47.290001) (end 106.644203 47.29) (width 0.2) (layer "B.Cu") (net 26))
 (segment (start 153.11 51.008477) (end 151.248478 52.869999) (width 0.2) (layer "F.Cu") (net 2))
 (segment (start 121.953462 34.389997) (end 149.309997 34.389997) (width 0.2) (layer "F.Cu") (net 2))
 (segment (start 114.752517 38.207999) (end 118.13546 38.207999) (width 0.2) (layer "F.Cu") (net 2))
 (segment (start 149.309997 34.389997) (end 153.11 38.19) (width 0.2) (layer "F.Cu") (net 2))
 (segment (start 153.11 38.19) (end 153.11 51.008477) (width 0.2) (layer "F.Cu") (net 2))
 (segment (start 118.13546 38.207999) (end 121.953462 34.389997) (width 0.2) (layer "F.Cu") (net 2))
 (segment (start 151.248476 37.528476) (end 148.909999 35.189999) (width 0.2) (layer "F.Cu") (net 7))
 (segment (start 148.909999 35.189999) (end 122.284832 35.189999) (width 0.2) (layer "F.Cu") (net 7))
 (segment (start 116.72683 40.748001) (end 114.752517 40.748001) (width 0.2) (layer "F.Cu") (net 7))
 (segment (start 151.248476 40.670001) (end 151.248476 37.528476) (width 0.2) (layer "F.Cu") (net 7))
 (segment (start 122.284832 35.189999) (end 116.72683 40.748001) (width 0.2) (layer "F.Cu") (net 7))
 (segment (start 147.710002 35.590002) (end 122.450515 35.590002) (width 0.2) (layer "F.Cu") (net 6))
 (segment (start 148.71 36.59) (end 147.710002 35.590002) (width 0.2) (layer "F.Cu") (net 6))
 (segment (start 151.248476 43.210001) (end 149.330001 43.210001) (width 0.2) (layer "F.Cu") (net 6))
 (segment (start 148.71 42.59) (end 148.71 36.59) (width 0.2) (layer "F.Cu") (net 6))
 (segment (start 122.450515 35.590002) (end 114.752517 43.288) (width 0.2) (layer "F.Cu") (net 6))
 (segment (start 149.330001 43.210001) (end 148.71 42.59) (width 0.2) (layer "F.Cu") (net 6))
 (segment (start 122.781887 36.390002) (end 132.06051 36.390002) (width 0.2) (layer "F.Cu") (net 8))
 (segment (start 114.752515 48.367998) (end 116.51 46.610513) (width 0.2) (layer "F.Cu") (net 8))
 (segment (start 116.51 46.610513) (end 116.51 42.661889) (width 0.2) (layer "F.Cu") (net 8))
 (segment (start 116.51 42.661889) (end 122.781887 36.390002) (width 0.2) (layer "F.Cu") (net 8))
 (segment (start 132.06051 36.390002) (end 134.108556 38.438048) (width 0.2) (layer "F.Cu") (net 8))
 (segment (start 134.108556 38.438048) (end 134.108556 40.670001) (width 0.2) (layer "F.Cu") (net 8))
 (segment (start 113.478515 49.634001) (end 113.478519 47.69) (width 0.2) (layer "F.Cu") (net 9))
 (segment (start 113.978519 47.19) (end 115.364827 47.19) (width 0.2) (layer "F.Cu") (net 9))
 (segment (start 113.478519 47.69) (end 113.978519 47.19) (width 0.2) (layer "F.Cu") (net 9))
 (segment (start 136.51 40.273806) (end 136.51 42.79) (width 0.2) (layer "F.Cu") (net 9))
 (segment (start 116.11 42.496203) (end 122.616201 35.990002) (width 0.2) (layer "F.Cu") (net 9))
 (segment (start 136.089999 43.210001) (end 134.108556 43.210001) (width 0.2) (layer "F.Cu") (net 9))
 (segment (start 132.226196 35.990002) (end 136.51 40.273806) (width 0.2) (layer "F.Cu") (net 9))
 (segment (start 115.364827 47.19) (end 116.11 46.444827) (width 0.2) (layer "F.Cu") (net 9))
 (segment (start 114.752515 50.908001) (end 113.478515 49.634001) (width 0.2) (layer "F.Cu") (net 9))
 (segment (start 122.616201 35.990002) (end 132.226196 35.990002) (width 0.2) (layer "F.Cu") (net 9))
 (segment (start 116.11 46.444827) (end 116.11 42.496203) (width 0.2) (layer "F.Cu") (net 9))
 (segment (start 136.51 42.79) (end 136.089999 43.210001) (width 0.2) (layer "F.Cu") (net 9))
 (segment (start 116.402314 53.448) (end 121.344314 58.39) (width 0.2) (layer "F.Cu") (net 3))
 (segment (start 149.11 50.79) (end 151.208475 50.79) (width 0.2) (layer "F.Cu") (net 3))
 (segment (start 141.51 58.39) (end 149.11 50.79) (width 0.2) (layer "F.Cu") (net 3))
 (segment (start 114.752516 53.448) (end 116.402314 53.448) (width 0.2) (layer "F.Cu") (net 3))
 (segment (start 151.248476 50.830001) (end 151.248476 50.330002) (width 0.2) (layer "F.Cu") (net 3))
 (segment (start 151.208475 50.79) (end 151.248476 50.830001) (width 0.2) (layer "F.Cu") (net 3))
 (segment (start 121.344314 58.39) (end 141.51 58.39) (width 0.2) (layer "F.Cu") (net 3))
 (segment (start 149.110001 34.790001) (end 122.119144 34.790001) (width 0.2) (layer "F.Cu") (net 4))
 (segment (start 117.519144 39.390001) (end 114.110001 39.390001) (width 0.2) (layer "F.Cu") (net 4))
 (segment (start 152.71 38.39) (end 149.110001 34.790001) (width 0.2) (layer "F.Cu") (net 4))
 (segment (start 151.248474 48.29) (end 152.71 46.828474) (width 0.2) (layer "F.Cu") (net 4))
 (segment (start 114.110001 39.390001) (end 110.71 35.99) (width 0.2) (layer "F.Cu") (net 4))
 (segment (start 122.119144 34.790001) (end 117.519144 39.390001) (width 0.2) (layer "F.Cu") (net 4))
 (segment (start 152.71 46.828474) (end 152.71 38.39) (width 0.2) (layer "F.Cu") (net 4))
 (segment (start 96.650515 35.99) (end 94.432515 38.208) (width 0.2) (layer "F.Cu") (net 4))
 (segment (start 110.71 35.99) (end 96.650515 35.99) (width 0.2) (layer "F.Cu") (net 4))
 (segment (start 136.878514 48.29) (end 134.108556 48.29) (width 0.2) (layer "F.Cu") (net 11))
 (via (at 136.878514 48.29) (size 0.8) (drill 0.4) (layers "F.Cu" "B.Cu") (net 11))
 (segment (start 139.409887 34.59) (end 102.564829 34.59) (width 0.2) (layer "B.Cu") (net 11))
 (segment (start 136.878514 48.29) (end 140.478516 44.689998) (width 0.2) (layer "B.Cu") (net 11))
 (segment (start 140.478516 44.689998) (end 140.478516 35.658629) (width 0.2) (layer "B.Cu") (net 11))
 (segment (start 96.40683 40.748) (end 94.432517 40.748) (width 0.2) (layer "B.Cu") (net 11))
 (segment (start 140.478516 35.658629) (end 139.409887 34.59) (width 0.2) (layer "B.Cu") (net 11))
 (segment (start 102.564829 34.59) (end 96.40683 40.748) (width 0.2) (layer "B.Cu") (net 11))
 (segment (start 134.148554 45.79) (end 134.108555 45.750001) (width 0.2) (layer "F.Cu") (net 10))
 (segment (start 136.91 45.79) (end 134.148554 45.79) (width 0.2) (layer "F.Cu") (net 10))
 (via (at 136.91 45.79) (size 0.8) (drill 0.4) (layers "F.Cu" "B.Cu") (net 10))
 (segment (start 140.078516 42.621484) (end 140.078516 35.824315) (width 0.2) (layer "B.Cu") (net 10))
 (segment (start 140.078516 35.824315) (end 139.244201 34.99) (width 0.2) (layer "B.Cu") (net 10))
 (segment (start 102.730515 34.99) (end 94.432517 43.288) (width 0.2) (layer "B.Cu") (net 10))
 (segment (start 139.244201 34.99) (end 102.730515 34.99) (width 0.2) (layer "B.Cu") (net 10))
 (segment (start 136.91 45.79) (end 140.078516 42.621484) (width 0.2) (layer "B.Cu") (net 10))
 (segment (start 94.432516 48.367999) (end 95.71 47.090515) (width 0.2) (layer "B.Cu") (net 16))
 (segment (start 102.896201 35.39) (end 139.078516 35.39) (width 0.2) (layer "B.Cu") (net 16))
 (segment (start 139.678516 38.481422) (end 138.973224 39.186714) (width 0.2) (layer "B.Cu") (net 16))
 (segment (start 95.71 47.090515) (end 95.71 42.576201) (width 0.2) (layer "B.Cu") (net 16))
 (segment (start 139.678516 35.99) (end 139.678516 38.481422) (width 0.2) (layer "B.Cu") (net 16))
 (segment (start 95.71 42.576201) (end 102.896201 35.39) (width 0.2) (layer "B.Cu") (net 16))
 (segment (start 139.078516 35.39) (end 139.678516 35.99) (width 0.2) (layer "B.Cu") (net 16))
 (segment (start 96.11 42.741887) (end 103.061887 35.79) (width 0.2) (layer "B.Cu") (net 17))
 (segment (start 96.11 49.230514) (end 96.11 42.741887) (width 0.2) (layer "B.Cu") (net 17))
 (segment (start 133.487097 35.79) (end 136.871307 39.17421) (width 0.2) (layer "B.Cu") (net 17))
 (segment (start 94.432513 50.908001) (end 96.11 49.230514) (width 0.2) (layer "B.Cu") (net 17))
 (segment (start 103.061887 35.79) (end 133.487097 35.79) (width 0.2) (layer "B.Cu") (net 17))
 (segment (start 141.344314 57.99) (end 121.51 57.99) (width 0.2) (layer "F.Cu") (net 5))
 (segment (start 151.248476 45.750001) (end 149.349999 45.750001) (width 0.2) (layer "F.Cu") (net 5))
 (segment (start 149.349999 45.750001) (end 148.71 46.39) (width 0.2) (layer "F.Cu") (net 5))
 (segment (start 148.71 50.624314) (end 141.344314 57.99) (width 0.2) (layer "F.Cu") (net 5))
 (segment (start 121.51 57.99) (end 115.71 52.19) (width 0.2) (layer "F.Cu") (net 5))
 (segment (start 148.71 46.39) (end 148.71 50.624314) (width 0.2) (layer "F.Cu") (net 5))
 (segment (start 115.71 52.19) (end 95.690515 52.19) (width 0.2) (layer "F.Cu") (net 5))
 (segment (start 95.690515 52.19) (end 94.432515 53.448) (width 0.2) (layer "F.Cu") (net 5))
 (segment (start 155.31 51.45) (end 153.51 49.65) (width 1) (layer "B.Cu") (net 18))
 (segment (start 153.51 49.65) (end 153.51 43.19) (width 1) (layer "B.Cu") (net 18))
 (segment (start 153.51 43.19) (end 155.31 41.39) (width 1) (layer "B.Cu") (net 18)))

